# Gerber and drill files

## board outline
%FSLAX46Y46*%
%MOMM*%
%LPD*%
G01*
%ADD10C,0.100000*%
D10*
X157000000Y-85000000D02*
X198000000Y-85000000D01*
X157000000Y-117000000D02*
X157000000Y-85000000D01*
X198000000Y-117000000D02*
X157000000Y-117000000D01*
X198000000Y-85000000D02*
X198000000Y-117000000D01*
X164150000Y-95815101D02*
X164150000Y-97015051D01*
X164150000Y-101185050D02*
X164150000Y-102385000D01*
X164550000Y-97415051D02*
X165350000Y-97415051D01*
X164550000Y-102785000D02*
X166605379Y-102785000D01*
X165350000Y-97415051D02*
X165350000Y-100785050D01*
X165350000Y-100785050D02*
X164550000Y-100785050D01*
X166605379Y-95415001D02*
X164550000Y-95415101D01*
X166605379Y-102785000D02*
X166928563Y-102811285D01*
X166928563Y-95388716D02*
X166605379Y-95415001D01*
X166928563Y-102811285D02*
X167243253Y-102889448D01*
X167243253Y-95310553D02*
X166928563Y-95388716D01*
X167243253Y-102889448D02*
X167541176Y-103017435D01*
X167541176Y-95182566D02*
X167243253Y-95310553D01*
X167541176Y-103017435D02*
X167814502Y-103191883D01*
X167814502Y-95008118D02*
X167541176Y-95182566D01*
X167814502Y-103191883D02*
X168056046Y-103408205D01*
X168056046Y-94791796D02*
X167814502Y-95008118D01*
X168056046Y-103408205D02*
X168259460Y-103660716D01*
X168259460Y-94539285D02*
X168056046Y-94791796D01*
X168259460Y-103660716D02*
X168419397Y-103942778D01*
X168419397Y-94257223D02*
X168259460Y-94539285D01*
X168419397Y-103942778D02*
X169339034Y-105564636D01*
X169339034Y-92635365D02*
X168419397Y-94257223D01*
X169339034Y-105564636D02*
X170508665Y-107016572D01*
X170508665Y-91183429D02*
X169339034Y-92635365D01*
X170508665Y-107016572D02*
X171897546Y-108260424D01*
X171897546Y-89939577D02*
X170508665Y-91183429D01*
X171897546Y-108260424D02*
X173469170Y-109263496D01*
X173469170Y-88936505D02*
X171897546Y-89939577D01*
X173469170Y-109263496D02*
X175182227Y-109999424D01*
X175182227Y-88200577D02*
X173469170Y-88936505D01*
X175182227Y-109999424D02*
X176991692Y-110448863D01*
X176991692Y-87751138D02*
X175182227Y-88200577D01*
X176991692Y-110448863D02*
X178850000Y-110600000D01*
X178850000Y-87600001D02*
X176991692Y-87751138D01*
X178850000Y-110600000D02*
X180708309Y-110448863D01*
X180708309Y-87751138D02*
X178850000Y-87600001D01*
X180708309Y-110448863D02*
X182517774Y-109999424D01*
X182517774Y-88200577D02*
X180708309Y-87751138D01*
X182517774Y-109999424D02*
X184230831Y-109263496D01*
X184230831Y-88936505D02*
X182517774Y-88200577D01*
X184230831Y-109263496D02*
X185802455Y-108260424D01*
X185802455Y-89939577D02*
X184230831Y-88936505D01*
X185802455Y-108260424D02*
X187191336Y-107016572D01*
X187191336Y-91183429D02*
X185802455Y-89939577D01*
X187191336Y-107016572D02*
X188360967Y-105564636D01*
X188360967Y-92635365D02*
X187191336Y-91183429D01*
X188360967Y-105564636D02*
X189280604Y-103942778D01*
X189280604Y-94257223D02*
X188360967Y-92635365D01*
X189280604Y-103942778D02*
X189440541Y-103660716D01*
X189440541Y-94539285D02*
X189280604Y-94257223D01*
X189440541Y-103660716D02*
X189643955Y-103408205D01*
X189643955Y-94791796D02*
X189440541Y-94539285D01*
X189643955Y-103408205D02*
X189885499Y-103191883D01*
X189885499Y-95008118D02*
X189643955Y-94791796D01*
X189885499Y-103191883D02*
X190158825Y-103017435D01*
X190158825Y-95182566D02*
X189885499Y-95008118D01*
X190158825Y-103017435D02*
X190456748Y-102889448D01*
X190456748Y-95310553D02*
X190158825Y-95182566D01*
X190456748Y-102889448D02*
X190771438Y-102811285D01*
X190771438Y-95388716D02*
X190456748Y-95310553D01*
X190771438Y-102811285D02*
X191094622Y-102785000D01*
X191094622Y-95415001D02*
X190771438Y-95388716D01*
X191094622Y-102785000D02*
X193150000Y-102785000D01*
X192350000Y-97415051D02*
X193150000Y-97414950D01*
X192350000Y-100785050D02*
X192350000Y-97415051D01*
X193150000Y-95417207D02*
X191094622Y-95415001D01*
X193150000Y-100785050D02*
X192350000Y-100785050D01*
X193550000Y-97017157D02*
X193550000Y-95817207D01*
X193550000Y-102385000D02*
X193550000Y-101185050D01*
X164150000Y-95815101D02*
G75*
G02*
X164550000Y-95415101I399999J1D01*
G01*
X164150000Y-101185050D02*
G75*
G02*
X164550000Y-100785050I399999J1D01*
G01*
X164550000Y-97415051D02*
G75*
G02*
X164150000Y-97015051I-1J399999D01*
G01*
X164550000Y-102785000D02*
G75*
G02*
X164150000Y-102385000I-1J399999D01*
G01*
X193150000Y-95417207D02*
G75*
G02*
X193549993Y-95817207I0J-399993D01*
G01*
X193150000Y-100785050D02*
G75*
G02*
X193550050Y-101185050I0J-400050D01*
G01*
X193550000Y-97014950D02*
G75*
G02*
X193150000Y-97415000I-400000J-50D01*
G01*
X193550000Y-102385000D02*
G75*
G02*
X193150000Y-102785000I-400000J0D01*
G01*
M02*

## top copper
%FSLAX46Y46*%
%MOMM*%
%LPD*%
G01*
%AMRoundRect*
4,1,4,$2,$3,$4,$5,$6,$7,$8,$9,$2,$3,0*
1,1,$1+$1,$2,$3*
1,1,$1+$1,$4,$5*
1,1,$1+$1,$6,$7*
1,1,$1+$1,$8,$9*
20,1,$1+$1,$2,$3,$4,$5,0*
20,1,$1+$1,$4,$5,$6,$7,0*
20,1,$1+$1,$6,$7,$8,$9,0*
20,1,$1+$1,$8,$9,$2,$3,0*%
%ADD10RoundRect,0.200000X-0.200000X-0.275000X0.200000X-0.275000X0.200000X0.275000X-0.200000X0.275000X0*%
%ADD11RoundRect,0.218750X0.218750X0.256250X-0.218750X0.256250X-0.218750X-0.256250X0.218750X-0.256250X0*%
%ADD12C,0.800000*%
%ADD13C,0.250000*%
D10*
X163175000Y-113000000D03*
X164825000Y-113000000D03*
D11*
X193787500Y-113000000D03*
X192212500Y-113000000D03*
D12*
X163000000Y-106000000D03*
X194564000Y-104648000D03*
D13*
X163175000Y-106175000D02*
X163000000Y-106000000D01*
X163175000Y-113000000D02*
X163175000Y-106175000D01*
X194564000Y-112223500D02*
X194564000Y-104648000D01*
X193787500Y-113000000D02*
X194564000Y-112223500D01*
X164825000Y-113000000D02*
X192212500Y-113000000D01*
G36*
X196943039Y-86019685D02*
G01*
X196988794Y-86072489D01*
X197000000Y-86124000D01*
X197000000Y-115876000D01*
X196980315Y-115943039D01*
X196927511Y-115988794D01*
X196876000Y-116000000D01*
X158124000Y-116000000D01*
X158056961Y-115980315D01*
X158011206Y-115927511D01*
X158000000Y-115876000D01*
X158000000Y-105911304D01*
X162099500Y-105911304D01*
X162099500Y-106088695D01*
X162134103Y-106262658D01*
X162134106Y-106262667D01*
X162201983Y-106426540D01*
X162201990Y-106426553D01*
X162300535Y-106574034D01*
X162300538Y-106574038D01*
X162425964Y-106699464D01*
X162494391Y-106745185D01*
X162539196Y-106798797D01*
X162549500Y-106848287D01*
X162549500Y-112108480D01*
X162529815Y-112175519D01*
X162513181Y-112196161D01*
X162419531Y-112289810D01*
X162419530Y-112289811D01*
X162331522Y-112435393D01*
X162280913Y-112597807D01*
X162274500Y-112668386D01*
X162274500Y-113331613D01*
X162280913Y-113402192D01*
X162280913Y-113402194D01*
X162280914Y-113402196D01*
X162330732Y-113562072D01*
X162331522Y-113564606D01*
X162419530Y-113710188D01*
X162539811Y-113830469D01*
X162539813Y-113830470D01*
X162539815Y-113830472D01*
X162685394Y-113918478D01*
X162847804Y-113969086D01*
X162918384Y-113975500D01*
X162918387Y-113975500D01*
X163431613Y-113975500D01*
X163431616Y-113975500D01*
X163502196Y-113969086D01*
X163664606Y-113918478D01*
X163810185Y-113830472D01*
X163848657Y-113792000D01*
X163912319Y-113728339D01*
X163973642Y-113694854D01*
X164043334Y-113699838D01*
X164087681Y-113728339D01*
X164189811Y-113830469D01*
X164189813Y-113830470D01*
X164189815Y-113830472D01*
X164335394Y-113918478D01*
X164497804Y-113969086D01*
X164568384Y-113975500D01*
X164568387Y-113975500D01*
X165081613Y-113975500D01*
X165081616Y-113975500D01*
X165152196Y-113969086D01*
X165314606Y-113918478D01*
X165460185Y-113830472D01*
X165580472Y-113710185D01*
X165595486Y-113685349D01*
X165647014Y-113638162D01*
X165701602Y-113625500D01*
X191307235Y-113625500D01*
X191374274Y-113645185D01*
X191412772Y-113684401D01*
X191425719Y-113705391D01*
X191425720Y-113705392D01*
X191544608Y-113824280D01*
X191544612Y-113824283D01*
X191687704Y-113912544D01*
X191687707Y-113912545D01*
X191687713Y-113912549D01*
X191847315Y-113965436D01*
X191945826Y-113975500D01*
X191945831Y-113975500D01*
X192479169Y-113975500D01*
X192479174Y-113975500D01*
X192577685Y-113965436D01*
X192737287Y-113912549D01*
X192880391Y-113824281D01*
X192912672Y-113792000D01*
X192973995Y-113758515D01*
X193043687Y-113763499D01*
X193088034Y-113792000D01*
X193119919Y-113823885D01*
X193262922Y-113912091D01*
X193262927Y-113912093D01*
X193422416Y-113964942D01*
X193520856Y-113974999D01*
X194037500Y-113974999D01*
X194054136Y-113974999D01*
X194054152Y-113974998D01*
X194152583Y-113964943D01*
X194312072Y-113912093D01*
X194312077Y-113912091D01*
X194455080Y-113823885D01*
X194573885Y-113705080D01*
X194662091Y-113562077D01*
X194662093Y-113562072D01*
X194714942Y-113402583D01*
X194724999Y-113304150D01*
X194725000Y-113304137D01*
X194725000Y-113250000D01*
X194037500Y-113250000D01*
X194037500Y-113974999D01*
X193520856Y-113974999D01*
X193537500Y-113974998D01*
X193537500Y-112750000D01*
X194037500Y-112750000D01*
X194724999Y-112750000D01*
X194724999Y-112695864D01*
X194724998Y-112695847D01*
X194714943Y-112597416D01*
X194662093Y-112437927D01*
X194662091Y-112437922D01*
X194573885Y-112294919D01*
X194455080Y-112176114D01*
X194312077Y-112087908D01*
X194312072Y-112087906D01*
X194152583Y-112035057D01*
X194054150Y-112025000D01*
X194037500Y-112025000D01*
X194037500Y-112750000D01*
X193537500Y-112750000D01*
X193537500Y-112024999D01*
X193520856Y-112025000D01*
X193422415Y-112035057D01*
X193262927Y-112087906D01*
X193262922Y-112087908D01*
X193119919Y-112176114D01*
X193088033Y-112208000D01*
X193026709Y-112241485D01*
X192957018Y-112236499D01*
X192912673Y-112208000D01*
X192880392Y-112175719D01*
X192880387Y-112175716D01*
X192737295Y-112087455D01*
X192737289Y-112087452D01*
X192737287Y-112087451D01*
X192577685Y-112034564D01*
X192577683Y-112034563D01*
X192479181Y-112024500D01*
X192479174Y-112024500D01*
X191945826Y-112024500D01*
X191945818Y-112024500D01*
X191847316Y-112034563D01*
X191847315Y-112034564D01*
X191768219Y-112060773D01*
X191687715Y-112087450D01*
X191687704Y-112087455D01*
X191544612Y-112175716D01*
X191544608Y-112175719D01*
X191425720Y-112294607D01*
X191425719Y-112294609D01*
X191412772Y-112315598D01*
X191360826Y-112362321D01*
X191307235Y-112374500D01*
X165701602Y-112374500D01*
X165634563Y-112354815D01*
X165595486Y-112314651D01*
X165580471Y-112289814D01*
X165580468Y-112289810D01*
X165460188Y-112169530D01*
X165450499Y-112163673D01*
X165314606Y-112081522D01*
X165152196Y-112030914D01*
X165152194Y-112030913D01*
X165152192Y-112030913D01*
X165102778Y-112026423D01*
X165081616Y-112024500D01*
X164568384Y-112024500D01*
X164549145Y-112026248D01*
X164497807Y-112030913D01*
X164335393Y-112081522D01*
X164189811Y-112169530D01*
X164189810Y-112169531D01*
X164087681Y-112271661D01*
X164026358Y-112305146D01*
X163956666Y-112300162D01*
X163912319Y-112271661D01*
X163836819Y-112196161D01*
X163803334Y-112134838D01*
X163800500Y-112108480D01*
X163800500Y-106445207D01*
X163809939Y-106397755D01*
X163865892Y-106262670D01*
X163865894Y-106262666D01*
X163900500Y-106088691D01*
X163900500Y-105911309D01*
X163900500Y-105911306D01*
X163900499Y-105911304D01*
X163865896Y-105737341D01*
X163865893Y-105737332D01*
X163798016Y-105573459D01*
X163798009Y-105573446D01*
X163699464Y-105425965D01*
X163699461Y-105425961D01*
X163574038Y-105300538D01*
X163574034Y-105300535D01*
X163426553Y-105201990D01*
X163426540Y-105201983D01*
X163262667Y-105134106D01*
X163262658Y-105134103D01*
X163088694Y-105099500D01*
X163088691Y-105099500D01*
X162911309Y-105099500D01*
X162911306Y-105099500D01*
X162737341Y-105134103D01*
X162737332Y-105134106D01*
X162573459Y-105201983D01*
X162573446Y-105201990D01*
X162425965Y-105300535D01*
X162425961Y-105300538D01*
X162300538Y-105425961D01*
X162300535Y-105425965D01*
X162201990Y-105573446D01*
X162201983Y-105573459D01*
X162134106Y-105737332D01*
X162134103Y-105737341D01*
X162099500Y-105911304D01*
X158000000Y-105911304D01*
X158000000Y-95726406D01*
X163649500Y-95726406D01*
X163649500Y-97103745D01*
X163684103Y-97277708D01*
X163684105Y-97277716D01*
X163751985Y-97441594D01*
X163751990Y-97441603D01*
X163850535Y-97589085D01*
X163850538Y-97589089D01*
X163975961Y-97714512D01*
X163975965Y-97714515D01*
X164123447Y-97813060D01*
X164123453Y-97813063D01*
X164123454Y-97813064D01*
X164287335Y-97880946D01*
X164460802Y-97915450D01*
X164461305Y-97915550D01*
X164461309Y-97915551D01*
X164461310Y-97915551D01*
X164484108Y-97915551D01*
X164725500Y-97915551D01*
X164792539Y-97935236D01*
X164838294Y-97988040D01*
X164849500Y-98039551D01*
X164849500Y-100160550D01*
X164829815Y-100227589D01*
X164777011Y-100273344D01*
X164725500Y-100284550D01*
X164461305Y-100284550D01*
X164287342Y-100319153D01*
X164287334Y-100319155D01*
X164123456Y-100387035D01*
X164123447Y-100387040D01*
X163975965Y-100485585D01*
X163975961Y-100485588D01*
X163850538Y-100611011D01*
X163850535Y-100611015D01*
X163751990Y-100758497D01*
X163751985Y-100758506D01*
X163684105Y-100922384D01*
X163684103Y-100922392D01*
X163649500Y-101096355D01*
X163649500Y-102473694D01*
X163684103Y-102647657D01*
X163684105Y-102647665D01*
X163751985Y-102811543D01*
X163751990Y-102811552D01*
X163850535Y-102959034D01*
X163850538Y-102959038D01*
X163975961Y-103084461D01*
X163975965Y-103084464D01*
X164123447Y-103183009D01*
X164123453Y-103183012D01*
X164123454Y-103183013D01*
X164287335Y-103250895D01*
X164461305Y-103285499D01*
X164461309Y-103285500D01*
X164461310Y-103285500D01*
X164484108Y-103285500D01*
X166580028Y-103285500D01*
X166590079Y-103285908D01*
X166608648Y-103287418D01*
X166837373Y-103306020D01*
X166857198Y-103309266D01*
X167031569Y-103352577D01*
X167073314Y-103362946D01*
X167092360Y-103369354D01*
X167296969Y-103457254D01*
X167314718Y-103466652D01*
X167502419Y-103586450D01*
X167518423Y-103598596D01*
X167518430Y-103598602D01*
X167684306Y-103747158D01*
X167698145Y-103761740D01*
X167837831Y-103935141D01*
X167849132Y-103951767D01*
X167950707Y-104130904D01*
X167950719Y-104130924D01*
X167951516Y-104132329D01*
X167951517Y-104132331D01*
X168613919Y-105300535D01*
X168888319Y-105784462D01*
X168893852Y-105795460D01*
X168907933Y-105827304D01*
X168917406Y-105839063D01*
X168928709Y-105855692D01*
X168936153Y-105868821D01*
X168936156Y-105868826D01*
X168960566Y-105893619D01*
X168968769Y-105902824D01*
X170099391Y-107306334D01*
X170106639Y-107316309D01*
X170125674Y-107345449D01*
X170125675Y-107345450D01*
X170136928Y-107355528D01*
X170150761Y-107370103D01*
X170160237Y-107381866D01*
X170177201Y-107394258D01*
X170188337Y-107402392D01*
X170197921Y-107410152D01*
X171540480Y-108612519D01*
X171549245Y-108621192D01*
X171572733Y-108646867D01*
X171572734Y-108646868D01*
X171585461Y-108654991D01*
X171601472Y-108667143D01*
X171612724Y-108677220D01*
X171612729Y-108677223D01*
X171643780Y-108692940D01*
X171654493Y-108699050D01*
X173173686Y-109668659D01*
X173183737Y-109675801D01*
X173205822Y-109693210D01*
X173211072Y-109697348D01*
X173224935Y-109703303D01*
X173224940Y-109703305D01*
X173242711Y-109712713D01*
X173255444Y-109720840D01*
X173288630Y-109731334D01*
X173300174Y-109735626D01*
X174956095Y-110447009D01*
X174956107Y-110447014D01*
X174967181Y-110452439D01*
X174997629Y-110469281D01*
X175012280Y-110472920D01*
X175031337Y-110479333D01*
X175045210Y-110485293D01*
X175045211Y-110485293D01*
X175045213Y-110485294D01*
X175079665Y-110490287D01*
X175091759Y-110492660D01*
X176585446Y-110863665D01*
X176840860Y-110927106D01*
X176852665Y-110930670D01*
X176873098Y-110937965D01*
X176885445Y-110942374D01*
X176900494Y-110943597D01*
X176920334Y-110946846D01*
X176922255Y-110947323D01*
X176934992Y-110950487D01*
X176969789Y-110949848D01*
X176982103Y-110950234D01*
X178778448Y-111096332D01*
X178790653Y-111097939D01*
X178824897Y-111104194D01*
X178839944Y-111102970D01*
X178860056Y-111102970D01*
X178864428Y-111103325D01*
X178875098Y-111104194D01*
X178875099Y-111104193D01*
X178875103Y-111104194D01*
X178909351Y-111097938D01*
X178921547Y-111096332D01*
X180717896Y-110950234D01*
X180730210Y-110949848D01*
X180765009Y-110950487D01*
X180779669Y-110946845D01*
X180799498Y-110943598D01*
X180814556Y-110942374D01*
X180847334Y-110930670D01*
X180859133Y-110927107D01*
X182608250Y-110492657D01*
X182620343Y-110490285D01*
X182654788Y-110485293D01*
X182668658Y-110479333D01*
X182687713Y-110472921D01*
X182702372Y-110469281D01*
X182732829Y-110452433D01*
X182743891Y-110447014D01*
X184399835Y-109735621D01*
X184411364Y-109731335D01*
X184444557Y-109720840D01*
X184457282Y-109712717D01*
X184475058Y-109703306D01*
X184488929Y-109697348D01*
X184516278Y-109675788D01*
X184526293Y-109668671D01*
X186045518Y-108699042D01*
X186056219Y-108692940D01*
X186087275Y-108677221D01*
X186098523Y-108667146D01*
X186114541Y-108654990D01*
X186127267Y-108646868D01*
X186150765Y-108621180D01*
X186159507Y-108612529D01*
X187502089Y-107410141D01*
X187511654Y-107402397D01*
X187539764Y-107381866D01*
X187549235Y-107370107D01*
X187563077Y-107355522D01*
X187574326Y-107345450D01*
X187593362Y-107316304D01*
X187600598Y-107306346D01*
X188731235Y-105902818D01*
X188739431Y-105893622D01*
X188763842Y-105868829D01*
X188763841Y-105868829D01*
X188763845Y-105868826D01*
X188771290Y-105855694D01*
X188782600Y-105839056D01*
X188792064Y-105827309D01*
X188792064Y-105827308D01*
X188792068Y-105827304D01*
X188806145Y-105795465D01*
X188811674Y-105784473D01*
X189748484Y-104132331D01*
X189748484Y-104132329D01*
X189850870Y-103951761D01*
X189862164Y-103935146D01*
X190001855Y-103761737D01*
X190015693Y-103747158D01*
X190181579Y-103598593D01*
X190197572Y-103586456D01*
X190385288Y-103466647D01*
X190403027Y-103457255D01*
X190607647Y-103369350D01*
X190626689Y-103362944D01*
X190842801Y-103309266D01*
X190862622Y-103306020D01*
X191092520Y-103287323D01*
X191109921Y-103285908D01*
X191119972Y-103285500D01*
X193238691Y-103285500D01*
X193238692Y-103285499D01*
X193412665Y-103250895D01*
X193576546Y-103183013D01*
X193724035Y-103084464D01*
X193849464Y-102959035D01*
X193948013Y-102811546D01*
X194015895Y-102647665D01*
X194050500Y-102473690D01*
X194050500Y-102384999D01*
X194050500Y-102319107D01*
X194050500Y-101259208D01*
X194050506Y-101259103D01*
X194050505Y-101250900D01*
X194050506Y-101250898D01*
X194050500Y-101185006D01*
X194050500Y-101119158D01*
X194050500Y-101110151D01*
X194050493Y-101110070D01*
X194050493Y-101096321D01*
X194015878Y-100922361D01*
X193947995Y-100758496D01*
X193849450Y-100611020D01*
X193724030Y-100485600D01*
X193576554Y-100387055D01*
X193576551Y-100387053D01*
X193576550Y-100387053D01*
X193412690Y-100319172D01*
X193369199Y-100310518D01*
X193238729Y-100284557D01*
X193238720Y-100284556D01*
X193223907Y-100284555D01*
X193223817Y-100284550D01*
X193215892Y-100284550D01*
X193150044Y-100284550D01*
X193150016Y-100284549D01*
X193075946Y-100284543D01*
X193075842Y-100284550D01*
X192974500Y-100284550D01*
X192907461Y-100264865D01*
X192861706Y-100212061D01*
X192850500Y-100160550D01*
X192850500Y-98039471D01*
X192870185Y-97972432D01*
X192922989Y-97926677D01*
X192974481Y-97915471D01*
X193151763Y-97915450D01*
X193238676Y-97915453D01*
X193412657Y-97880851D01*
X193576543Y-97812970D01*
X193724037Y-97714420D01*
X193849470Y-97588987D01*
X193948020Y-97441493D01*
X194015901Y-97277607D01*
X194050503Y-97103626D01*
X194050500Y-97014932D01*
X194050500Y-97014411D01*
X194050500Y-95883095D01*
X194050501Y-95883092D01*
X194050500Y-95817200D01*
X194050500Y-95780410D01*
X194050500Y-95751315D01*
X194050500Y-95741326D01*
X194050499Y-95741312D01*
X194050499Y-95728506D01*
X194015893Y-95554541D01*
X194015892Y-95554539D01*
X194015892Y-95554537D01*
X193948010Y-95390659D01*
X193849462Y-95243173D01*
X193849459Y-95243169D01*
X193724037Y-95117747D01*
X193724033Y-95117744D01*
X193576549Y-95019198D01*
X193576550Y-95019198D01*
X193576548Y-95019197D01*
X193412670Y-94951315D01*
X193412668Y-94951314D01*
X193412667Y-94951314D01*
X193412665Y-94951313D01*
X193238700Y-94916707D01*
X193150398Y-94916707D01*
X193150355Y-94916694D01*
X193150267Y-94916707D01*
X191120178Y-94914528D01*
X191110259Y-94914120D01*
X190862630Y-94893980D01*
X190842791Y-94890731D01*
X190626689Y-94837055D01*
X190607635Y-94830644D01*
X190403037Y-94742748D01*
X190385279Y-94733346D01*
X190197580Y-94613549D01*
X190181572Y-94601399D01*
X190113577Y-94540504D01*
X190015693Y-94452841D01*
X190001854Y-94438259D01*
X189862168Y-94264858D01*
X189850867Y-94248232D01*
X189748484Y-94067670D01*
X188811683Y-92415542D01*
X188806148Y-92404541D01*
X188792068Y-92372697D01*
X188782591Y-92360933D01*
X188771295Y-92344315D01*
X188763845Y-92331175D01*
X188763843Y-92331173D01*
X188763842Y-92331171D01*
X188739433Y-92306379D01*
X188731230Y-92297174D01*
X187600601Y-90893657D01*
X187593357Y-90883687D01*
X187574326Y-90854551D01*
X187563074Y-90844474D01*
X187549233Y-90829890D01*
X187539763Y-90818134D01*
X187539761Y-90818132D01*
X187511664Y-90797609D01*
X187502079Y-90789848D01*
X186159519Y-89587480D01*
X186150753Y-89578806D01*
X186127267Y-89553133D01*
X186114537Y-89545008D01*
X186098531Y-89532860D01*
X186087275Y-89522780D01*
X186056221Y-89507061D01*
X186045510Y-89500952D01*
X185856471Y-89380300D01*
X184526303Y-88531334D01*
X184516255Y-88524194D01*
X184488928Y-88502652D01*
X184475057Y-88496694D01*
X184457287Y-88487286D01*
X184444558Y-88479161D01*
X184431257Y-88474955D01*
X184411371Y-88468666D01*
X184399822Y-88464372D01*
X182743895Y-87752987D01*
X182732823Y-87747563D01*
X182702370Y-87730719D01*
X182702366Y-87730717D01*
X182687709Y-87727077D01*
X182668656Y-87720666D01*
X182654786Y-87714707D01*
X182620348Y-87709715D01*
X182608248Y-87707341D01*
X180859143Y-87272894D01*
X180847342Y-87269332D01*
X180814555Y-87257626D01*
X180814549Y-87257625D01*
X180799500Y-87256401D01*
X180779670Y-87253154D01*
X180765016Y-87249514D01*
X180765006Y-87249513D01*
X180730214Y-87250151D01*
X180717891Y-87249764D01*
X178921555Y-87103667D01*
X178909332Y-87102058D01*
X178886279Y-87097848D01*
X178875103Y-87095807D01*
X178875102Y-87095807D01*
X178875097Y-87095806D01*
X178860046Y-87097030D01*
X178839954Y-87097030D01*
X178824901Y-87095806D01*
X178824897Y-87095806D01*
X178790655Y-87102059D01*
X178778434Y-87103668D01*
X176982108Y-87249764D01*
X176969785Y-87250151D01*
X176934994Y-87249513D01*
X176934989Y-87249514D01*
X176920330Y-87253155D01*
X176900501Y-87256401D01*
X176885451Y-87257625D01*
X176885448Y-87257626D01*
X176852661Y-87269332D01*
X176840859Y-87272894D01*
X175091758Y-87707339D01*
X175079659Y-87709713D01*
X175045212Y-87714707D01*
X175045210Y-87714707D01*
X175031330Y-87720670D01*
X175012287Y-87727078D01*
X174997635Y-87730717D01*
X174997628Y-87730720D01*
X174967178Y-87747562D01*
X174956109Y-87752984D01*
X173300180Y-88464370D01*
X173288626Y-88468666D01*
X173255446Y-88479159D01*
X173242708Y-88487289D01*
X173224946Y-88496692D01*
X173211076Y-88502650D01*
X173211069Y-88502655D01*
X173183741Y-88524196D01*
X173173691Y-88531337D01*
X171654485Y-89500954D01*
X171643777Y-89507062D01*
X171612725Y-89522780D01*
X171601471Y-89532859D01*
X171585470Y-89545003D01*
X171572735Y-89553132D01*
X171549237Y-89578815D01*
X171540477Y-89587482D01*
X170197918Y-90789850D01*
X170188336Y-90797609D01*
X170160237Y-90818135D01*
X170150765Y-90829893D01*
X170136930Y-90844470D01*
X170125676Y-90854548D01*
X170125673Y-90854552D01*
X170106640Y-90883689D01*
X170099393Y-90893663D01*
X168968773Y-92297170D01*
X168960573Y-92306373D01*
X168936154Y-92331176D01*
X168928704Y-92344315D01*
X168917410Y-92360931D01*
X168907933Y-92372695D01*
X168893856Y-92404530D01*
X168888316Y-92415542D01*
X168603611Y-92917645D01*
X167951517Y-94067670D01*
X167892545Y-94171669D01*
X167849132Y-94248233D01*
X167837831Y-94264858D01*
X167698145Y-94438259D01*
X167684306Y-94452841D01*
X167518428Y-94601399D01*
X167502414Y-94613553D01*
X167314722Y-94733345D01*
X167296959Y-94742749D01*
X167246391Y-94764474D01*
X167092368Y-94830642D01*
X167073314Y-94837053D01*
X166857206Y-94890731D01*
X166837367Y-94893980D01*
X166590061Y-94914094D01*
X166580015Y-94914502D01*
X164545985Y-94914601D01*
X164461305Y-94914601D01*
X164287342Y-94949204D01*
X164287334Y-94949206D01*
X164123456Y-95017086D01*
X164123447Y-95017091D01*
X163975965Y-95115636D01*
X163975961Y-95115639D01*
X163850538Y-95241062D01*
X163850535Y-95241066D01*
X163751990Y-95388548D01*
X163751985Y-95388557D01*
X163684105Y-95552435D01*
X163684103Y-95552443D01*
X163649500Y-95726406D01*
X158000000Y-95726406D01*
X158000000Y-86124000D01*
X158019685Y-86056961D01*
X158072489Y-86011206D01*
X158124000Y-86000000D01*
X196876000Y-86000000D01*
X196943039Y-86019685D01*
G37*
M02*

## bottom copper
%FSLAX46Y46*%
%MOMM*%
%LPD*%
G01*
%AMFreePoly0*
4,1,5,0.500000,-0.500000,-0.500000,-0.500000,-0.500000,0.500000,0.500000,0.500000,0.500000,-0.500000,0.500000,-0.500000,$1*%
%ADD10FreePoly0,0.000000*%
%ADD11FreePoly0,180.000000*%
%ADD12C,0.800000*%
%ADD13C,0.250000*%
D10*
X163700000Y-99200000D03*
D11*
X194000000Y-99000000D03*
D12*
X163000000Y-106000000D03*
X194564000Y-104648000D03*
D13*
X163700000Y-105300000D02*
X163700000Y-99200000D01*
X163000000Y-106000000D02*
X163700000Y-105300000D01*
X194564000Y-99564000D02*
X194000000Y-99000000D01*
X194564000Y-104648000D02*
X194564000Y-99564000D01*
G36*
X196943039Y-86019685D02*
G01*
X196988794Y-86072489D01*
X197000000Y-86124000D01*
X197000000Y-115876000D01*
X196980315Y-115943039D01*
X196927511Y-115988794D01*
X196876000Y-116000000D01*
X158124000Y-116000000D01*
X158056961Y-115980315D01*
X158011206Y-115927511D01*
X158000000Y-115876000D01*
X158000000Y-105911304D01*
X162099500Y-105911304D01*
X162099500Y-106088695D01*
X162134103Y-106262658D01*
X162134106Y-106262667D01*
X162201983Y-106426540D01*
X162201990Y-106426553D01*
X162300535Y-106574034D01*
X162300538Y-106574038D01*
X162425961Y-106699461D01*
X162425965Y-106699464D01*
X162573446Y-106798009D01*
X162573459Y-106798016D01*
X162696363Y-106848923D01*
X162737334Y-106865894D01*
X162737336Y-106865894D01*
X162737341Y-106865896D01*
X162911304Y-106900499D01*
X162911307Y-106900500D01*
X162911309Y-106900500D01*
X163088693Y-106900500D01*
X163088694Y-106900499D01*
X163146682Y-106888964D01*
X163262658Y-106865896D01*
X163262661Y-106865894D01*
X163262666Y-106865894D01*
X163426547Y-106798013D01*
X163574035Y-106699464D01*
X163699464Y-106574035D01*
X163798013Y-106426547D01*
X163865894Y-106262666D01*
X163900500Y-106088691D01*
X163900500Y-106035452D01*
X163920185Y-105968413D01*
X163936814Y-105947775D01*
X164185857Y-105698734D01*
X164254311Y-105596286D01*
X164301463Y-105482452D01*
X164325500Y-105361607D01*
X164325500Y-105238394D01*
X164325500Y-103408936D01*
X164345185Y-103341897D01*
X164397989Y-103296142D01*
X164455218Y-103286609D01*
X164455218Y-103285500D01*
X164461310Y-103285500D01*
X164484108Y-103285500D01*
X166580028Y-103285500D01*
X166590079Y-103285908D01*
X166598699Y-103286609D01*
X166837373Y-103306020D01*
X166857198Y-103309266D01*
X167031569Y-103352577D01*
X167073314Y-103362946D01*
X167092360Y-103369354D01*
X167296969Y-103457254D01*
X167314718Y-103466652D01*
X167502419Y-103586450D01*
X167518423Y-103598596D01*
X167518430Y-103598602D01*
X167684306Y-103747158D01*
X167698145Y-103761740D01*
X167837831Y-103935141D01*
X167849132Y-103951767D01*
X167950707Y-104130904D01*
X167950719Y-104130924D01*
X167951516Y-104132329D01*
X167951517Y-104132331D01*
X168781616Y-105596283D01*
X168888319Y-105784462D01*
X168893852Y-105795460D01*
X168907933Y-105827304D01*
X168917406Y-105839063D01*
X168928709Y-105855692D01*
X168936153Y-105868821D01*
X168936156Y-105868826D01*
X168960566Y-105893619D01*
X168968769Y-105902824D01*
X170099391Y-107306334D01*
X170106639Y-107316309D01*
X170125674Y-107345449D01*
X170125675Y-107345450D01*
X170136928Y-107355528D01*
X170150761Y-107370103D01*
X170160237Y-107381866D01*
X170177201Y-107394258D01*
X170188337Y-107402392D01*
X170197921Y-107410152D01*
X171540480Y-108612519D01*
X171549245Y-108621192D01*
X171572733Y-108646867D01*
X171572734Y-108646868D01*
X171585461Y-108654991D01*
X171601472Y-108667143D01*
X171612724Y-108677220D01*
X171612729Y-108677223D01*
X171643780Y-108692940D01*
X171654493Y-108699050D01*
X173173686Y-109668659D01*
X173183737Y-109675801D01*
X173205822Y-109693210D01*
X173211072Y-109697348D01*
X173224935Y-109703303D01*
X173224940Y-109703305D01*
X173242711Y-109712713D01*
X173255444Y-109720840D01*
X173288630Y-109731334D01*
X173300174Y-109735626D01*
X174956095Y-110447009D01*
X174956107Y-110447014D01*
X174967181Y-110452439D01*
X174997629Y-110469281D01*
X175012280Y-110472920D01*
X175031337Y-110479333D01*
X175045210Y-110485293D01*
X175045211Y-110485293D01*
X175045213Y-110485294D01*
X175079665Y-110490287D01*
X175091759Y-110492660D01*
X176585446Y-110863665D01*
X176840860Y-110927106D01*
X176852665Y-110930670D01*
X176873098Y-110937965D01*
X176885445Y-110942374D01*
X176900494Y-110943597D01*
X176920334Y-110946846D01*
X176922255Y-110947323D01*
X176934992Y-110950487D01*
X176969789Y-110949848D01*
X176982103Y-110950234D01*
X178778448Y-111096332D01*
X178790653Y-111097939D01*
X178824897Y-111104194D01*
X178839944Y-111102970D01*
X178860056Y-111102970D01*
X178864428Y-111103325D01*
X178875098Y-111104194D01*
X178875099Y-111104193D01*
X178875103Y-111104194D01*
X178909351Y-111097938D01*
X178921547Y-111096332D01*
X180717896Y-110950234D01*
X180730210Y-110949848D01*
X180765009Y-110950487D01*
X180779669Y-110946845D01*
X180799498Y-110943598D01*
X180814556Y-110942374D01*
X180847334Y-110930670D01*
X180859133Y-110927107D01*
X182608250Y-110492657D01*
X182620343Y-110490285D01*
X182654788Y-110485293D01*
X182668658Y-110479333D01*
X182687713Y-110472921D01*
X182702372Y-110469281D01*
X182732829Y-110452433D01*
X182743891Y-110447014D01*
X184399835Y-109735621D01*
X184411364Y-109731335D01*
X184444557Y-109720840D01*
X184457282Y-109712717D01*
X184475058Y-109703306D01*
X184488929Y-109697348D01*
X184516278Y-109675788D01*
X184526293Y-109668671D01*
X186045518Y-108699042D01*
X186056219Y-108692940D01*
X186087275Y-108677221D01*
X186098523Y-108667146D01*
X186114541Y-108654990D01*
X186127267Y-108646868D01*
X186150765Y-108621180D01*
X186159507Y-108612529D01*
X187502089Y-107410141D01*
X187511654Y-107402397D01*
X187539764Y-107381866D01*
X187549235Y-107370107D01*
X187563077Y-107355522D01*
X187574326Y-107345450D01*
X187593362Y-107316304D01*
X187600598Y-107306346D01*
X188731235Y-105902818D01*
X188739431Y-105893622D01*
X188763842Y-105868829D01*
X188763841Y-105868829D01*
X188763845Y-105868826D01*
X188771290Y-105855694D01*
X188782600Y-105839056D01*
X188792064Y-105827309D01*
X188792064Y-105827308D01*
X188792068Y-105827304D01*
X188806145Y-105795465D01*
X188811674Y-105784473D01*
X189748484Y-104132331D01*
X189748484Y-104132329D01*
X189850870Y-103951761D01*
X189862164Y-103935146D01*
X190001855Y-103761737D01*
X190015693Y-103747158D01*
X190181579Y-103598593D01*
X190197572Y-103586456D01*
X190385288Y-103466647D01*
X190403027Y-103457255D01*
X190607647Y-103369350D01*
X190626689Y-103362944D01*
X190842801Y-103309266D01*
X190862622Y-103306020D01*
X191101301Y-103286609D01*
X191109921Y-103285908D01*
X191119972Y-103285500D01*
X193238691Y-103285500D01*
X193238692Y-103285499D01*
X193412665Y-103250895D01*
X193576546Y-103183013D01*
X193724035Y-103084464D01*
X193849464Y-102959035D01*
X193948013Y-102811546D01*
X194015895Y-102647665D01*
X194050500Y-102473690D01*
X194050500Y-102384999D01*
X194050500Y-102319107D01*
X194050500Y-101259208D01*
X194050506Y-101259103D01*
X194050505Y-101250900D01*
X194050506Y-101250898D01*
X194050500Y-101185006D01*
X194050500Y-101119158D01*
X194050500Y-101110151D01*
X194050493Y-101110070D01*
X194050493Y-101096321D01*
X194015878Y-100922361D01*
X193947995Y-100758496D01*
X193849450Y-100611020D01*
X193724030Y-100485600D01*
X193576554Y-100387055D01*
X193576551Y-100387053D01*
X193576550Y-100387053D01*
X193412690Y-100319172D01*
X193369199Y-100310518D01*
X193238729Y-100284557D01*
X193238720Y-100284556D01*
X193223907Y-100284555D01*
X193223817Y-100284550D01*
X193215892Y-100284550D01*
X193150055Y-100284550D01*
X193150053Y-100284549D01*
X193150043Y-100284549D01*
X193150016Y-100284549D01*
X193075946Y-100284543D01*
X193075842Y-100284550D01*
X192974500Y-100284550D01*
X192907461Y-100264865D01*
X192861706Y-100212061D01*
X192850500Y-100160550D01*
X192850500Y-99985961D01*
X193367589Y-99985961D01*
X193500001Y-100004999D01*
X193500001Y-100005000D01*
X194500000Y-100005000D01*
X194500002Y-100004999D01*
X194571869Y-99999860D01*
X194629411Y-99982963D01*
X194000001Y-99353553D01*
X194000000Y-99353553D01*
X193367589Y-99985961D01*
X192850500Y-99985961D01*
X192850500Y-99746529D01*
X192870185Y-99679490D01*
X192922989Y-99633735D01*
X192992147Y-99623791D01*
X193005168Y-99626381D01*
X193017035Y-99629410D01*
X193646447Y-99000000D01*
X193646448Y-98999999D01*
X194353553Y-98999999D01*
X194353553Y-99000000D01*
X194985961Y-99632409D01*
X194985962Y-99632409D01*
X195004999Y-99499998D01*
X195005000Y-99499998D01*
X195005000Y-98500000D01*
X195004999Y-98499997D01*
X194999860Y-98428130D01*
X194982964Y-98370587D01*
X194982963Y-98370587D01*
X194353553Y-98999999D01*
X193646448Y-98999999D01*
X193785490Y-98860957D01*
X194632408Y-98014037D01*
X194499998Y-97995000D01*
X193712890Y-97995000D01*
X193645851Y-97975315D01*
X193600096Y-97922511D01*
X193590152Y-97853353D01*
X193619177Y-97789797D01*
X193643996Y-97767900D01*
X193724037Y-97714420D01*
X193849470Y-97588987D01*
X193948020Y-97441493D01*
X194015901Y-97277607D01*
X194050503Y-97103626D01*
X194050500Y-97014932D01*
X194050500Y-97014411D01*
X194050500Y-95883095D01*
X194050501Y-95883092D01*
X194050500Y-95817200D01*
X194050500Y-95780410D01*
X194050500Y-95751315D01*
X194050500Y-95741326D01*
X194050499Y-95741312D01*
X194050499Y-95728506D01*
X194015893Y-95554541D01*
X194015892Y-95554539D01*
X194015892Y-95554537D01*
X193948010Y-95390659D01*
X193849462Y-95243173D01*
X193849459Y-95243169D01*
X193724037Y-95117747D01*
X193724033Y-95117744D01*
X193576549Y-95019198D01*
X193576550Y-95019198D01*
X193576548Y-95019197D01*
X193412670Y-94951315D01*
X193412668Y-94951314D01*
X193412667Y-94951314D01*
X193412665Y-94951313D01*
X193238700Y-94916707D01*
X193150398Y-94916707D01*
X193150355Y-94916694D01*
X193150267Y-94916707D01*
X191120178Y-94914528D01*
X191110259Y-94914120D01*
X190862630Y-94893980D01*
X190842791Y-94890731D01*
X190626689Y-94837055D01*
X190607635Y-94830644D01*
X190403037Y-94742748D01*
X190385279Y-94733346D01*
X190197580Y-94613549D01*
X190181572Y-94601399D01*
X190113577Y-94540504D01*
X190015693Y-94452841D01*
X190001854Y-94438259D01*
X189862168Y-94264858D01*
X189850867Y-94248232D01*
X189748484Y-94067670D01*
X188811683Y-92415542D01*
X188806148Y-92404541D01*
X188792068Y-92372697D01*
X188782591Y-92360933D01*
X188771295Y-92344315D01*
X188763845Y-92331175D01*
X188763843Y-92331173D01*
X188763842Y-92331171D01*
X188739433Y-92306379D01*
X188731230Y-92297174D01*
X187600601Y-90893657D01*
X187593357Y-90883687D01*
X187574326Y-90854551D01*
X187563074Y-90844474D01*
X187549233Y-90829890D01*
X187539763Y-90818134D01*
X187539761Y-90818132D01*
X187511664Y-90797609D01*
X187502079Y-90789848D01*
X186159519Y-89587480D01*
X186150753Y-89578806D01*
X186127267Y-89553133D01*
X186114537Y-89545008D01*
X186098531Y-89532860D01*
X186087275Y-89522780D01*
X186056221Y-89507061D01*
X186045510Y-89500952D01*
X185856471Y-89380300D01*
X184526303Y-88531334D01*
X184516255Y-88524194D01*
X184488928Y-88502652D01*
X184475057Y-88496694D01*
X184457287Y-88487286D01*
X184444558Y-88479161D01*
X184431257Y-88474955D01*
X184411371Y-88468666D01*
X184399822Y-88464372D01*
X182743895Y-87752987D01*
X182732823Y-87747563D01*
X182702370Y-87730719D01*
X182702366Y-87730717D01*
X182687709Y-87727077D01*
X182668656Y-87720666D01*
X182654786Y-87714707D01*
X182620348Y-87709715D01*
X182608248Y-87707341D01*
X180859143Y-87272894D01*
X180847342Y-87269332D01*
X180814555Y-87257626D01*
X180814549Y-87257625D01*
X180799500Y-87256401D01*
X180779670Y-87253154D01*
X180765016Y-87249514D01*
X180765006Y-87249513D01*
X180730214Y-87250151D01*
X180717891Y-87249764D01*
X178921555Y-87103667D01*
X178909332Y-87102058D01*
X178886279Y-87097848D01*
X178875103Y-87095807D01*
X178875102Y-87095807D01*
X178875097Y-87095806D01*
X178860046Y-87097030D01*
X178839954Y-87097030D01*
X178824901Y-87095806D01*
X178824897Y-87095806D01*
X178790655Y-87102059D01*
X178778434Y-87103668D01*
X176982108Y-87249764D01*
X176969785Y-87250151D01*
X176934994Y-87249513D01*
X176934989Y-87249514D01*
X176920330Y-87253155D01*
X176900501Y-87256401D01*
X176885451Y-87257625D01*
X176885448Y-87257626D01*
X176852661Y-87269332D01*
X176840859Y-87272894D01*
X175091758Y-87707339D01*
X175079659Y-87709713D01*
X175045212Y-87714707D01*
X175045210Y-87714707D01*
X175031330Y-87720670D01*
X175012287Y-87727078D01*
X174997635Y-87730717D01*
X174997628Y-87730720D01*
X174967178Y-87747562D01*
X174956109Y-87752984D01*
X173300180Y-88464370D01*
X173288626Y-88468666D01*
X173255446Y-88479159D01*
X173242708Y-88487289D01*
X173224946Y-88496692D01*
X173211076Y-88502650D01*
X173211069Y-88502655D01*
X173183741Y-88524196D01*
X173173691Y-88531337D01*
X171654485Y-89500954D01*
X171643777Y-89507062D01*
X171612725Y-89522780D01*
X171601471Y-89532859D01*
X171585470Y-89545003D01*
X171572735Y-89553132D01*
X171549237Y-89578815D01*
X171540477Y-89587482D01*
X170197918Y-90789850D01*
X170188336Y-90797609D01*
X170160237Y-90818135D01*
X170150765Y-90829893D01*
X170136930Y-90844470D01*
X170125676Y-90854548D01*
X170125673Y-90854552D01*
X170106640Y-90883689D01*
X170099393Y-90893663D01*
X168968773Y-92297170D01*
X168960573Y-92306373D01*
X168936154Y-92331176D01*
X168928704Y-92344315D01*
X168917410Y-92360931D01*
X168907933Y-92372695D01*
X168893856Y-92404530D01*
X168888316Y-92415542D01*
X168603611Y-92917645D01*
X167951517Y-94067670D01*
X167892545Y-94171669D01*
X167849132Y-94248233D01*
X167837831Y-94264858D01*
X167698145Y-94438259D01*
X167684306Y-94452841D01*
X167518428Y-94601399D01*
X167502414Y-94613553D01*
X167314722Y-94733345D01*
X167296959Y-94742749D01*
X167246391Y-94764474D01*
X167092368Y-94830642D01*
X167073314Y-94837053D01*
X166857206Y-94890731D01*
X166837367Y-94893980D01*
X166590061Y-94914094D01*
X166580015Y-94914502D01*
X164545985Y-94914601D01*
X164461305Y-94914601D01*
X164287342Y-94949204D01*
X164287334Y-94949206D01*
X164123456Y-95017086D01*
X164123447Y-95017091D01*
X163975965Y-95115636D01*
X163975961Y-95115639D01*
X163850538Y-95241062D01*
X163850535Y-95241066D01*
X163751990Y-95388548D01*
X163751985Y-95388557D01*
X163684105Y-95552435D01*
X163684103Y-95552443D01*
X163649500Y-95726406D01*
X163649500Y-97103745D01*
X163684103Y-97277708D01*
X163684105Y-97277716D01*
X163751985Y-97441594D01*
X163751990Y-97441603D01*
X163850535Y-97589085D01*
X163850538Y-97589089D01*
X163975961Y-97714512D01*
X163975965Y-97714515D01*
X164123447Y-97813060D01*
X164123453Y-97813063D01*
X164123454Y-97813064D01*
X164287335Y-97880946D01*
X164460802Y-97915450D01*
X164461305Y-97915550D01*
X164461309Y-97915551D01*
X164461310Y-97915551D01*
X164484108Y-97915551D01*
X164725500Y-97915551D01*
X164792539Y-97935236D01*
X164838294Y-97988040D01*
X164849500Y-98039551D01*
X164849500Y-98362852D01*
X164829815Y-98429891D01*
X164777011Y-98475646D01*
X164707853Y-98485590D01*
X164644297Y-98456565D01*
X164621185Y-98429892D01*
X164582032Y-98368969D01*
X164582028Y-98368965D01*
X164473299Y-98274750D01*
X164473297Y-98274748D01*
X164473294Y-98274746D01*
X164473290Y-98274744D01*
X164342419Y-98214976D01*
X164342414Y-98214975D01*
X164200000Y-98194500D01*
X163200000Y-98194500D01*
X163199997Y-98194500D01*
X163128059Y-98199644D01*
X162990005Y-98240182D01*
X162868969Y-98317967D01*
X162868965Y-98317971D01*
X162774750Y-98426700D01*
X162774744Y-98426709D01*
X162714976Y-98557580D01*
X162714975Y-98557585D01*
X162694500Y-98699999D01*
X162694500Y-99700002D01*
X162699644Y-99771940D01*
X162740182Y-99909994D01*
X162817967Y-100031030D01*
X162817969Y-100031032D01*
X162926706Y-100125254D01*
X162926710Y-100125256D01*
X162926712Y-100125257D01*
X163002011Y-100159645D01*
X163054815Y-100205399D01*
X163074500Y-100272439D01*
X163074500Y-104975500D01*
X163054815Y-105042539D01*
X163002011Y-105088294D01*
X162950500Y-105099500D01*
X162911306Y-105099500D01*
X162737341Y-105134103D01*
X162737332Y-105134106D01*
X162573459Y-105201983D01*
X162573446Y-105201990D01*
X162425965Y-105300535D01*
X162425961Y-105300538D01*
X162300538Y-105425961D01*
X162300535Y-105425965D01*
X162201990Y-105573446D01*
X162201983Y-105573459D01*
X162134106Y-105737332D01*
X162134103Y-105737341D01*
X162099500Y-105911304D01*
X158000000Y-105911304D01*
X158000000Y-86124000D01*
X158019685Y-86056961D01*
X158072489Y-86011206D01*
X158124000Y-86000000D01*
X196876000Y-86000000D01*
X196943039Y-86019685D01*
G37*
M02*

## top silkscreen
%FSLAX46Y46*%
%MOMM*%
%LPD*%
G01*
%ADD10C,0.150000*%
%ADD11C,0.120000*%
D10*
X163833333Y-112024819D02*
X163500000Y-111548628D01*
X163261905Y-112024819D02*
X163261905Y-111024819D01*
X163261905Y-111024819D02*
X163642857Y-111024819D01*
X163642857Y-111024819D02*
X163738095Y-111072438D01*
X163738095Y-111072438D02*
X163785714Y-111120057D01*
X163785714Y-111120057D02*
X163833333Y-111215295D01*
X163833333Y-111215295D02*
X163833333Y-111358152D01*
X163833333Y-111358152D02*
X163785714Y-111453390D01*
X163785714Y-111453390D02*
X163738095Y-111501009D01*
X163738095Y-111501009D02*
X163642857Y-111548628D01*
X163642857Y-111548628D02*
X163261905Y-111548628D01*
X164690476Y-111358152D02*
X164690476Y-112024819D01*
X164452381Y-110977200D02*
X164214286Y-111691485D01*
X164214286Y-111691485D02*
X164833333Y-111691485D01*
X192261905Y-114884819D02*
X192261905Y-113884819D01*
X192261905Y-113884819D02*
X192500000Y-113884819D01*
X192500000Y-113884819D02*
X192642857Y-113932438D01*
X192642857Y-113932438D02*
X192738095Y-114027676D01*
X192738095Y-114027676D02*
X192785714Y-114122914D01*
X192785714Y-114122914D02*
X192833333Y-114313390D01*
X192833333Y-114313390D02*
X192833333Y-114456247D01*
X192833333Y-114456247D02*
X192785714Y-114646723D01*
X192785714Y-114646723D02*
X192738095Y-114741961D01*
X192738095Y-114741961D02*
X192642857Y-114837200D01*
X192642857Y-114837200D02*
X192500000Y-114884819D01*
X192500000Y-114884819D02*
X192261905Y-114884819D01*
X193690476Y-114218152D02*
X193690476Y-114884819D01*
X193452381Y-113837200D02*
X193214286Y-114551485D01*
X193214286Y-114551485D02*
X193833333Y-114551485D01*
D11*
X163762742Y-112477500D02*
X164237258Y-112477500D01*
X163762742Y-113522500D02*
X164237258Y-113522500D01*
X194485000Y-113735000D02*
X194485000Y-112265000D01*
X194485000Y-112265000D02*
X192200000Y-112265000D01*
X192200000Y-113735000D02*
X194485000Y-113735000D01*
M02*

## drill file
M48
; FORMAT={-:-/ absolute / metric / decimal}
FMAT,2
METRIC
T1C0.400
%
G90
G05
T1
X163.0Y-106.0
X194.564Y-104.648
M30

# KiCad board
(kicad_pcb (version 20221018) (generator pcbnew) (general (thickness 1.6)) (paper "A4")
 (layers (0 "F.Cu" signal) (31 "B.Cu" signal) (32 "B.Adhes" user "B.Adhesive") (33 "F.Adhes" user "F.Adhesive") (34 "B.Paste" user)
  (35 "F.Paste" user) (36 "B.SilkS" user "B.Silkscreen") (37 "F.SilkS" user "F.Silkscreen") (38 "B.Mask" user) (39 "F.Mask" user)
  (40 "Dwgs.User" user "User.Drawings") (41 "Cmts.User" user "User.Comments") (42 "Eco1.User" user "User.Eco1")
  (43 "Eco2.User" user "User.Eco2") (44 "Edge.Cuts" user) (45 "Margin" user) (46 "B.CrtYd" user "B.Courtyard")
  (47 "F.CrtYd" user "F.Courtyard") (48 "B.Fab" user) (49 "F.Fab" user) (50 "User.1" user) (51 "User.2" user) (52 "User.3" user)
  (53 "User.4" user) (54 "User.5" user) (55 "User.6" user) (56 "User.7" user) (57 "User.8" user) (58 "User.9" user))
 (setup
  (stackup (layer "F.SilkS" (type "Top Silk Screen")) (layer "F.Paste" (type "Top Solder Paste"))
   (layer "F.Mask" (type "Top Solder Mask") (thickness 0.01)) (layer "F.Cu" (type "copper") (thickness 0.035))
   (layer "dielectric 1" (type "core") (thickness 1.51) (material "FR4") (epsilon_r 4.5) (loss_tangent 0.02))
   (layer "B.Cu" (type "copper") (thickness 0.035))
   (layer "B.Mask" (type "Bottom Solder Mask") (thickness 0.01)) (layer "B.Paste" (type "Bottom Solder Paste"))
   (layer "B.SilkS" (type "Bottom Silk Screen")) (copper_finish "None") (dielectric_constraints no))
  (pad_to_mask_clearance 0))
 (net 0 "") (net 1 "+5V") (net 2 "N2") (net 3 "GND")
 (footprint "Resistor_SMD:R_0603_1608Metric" (layer "F.Cu") (at 164 113)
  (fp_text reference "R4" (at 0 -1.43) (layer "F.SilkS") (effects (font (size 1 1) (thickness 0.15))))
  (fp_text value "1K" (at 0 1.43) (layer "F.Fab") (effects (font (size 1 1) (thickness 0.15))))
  (fp_line (start -0.237258 -0.5225) (end 0.237258 -0.5225) (stroke (width 0.12) (type solid)) (layer "F.SilkS"))
  (fp_line (start -0.237258 0.5225) (end 0.237258 0.5225) (stroke (width 0.12) (type solid)) (layer "F.SilkS"))
  (pad "1" smd roundrect (at -0.825 0) (size 0.8 0.95) (layers "F.Cu" "F.Paste" "F.Mask") (roundrect_rratio 0.25) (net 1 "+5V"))
  (pad "2" smd roundrect (at 0.825 0) (size 0.8 0.95) (layers "F.Cu" "F.Paste" "F.Mask") (roundrect_rratio 0.25) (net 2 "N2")))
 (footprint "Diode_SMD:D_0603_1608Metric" (layer "F.Cu") (at 193 113 180)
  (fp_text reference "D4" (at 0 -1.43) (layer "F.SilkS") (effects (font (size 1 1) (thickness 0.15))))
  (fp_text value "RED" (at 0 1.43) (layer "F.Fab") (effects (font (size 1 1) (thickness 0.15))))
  (fp_line (start -1.485 -0.735) (end -1.485 0.735) (stroke (width 0.12) (type solid)) (layer "F.SilkS"))
  (fp_line (start -1.485 0.735) (end 0.8 0.735) (stroke (width 0.12) (type solid)) (layer "F.SilkS"))
  (fp_line (start 0.8 -0.735) (end -1.485 -0.735) (stroke (width 0.12) (type solid)) (layer "F.SilkS"))
  (pad "1" smd roundrect (at -0.7875 0 180) (size 0.875 0.95) (layers "F.Cu" "F.Paste" "F.Mask") (roundrect_rratio 0.25) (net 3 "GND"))
  (pad "2" smd roundrect (at 0.7875 0 180) (size 0.875 0.95) (layers "F.Cu" "F.Paste" "F.Mask") (roundrect_rratio 0.25) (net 2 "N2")))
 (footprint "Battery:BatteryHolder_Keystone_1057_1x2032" (layer "B.Cu") (at 178.85 99.1)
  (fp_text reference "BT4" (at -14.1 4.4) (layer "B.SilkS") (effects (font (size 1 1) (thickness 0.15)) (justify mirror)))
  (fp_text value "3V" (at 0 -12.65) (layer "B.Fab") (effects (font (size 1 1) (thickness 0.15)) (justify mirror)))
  (fp_line (start -14.7 -3.284899) (end -14.7 -2.084949) (stroke (width 0.1) (type solid)) (layer "Edge.Cuts"))
  (fp_line (start -14.7 2.08505) (end -14.7 3.285) (stroke (width 0.1) (type solid)) (layer "Edge.Cuts"))
  (fp_line (start -14.3 -1.684949) (end -13.5 -1.684949) (stroke (width 0.1) (type solid)) (layer "Edge.Cuts"))
  (fp_line (start -14.3 3.685) (end -12.244621 3.685) (stroke (width 0.1) (type solid)) (layer "Edge.Cuts"))
  (fp_line (start -13.5 -1.684949) (end -13.5 1.68505) (stroke (width 0.1) (type solid)) (layer "Edge.Cuts"))
  (fp_line (start -13.5 1.68505) (end -14.3 1.68505) (stroke (width 0.1) (type solid)) (layer "Edge.Cuts"))
  (fp_line (start -12.244621 -3.684999) (end -14.3 -3.684899) (stroke (width 0.1) (type solid)) (layer "Edge.Cuts"))
  (fp_line (start -12.244621 3.685) (end -11.921437 3.711285) (stroke (width 0.1) (type solid)) (layer "Edge.Cuts"))
  (fp_line (start -11.921437 -3.711284) (end -12.244621 -3.684999) (stroke (width 0.1) (type solid)) (layer "Edge.Cuts"))
  (fp_line (start -11.921437 3.711285) (end -11.606747 3.789448) (stroke (width 0.1) (type solid)) (layer "Edge.Cuts"))
  (fp_line (start -11.606747 -3.789447) (end -11.921437 -3.711284) (stroke (width 0.1) (type solid)) (layer "Edge.Cuts"))
  (fp_line (start -11.606747 3.789448) (end -11.308824 3.917435) (stroke (width 0.1) (type solid)) (layer "Edge.Cuts"))
  (fp_line (start -11.308824 -3.917434) (end -11.606747 -3.789447) (stroke (width 0.1) (type solid)) (layer "Edge.Cuts"))
  (fp_line (start -11.308824 3.917435) (end -11.035498 4.091883) (stroke (width 0.1) (type solid)) (layer "Edge.Cuts"))
  (fp_line (start -11.035498 -4.091882) (end -11.308824 -3.917434) (stroke (width 0.1) (type solid)) (layer "Edge.Cuts"))
  (fp_line (start -11.035498 4.091883) (end -10.793954 4.308205) (stroke (width 0.1) (type solid)) (layer "Edge.Cuts"))
  (fp_line (start -10.793954 -4.308204) (end -11.035498 -4.091882) (stroke (width 0.1) (type solid)) (layer "Edge.Cuts"))
  (fp_line (start -10.793954 4.308205) (end -10.59054 4.560716) (stroke (width 0.1) (type solid)) (layer "Edge.Cuts"))
  (fp_line (start -10.59054 -4.560715) (end -10.793954 -4.308204) (stroke (width 0.1) (type solid)) (layer "Edge.Cuts"))
  (fp_line (start -10.59054 4.560716) (end -10.430603 4.842778) (stroke (width 0.1) (type solid)) (layer "Edge.Cuts"))
  (fp_line (start -10.430603 -4.842777) (end -10.59054 -4.560715) (stroke (width 0.1) (type solid)) (layer "Edge.Cuts"))
  (fp_line (start -10.430603 4.842778) (end -9.510966 6.464636) (stroke (width 0.1) (type solid)) (layer "Edge.Cuts"))
  (fp_line (start -9.510966 -6.464635) (end -10.430603 -4.842777) (stroke (width 0.1) (type solid)) (layer "Edge.Cuts"))
  (fp_line (start -9.510966 6.464636) (end -8.341335 7.916572) (stroke (width 0.1) (type solid)) (layer "Edge.Cuts"))
  (fp_line (start -8.341335 -7.916571) (end -9.510966 -6.464635) (stroke (width 0.1) (type solid)) (layer "Edge.Cuts"))
  (fp_line (start -8.341335 7.916572) (end -6.952454 9.160424) (stroke (width 0.1) (type solid)) (layer "Edge.Cuts"))
  (fp_line (start -6.952454 -9.160423) (end -8.341335 -7.916571) (stroke (width 0.1) (type solid)) (layer "Edge.Cuts"))
  (fp_line (start -6.952454 9.160424) (end -5.38083 10.163496) (stroke (width 0.1) (type solid)) (layer "Edge.Cuts"))
  (fp_line (start -5.38083 -10.163495) (end -6.952454 -9.160423) (stroke (width 0.1) (type solid)) (layer "Edge.Cuts"))
  (fp_line (start -5.38083 10.163496) (end -3.667773 10.899424) (stroke (width 0.1) (type solid)) (layer "Edge.Cuts"))
  (fp_line (start -3.667773 -10.899423) (end -5.38083 -10.163495) (stroke (width 0.1) (type solid)) (layer "Edge.Cuts"))
  (fp_line (start -3.667773 10.899424) (end -1.858308 11.348863) (stroke (width 0.1) (type solid)) (layer "Edge.Cuts"))
  (fp_line (start -1.858308 -11.348862) (end -3.667773 -10.899423) (stroke (width 0.1) (type solid)) (layer "Edge.Cuts"))
  (fp_line (start -1.858308 11.348863) (end 0 11.5) (stroke (width 0.1) (type solid)) (layer "Edge.Cuts"))
  (fp_line (start 0 -11.499999) (end -1.858308 -11.348862) (stroke (width 0.1) (type solid)) (layer "Edge.Cuts"))
  (fp_line (start 0 11.5) (end 1.858309 11.348863) (stroke (width 0.1) (type solid)) (layer "Edge.Cuts"))
  (fp_line (start 1.858309 -11.348862) (end 0 -11.499999) (stroke (width 0.1) (type solid)) (layer "Edge.Cuts"))
  (fp_line (start 1.858309 11.348863) (end 3.667774 10.899424) (stroke (width 0.1) (type solid)) (layer "Edge.Cuts"))
  (fp_line (start 3.667774 -10.899423) (end 1.858309 -11.348862) (stroke (width 0.1) (type solid)) (layer "Edge.Cuts"))
  (fp_line (start 3.667774 10.899424) (end 5.380831 10.163496) (stroke (width 0.1) (type solid)) (layer "Edge.Cuts"))
  (fp_line (start 5.380831 -10.163495) (end 3.667774 -10.899423) (stroke (width 0.1) (type solid)) (layer "Edge.Cuts"))
  (fp_line (start 5.380831 10.163496) (end 6.952455 9.160424) (stroke (width 0.1) (type solid)) (layer "Edge.Cuts"))
  (fp_line (start 6.952455 -9.160423) (end 5.380831 -10.163495) (stroke (width 0.1) (type solid)) (layer "Edge.Cuts"))
  (fp_line (start 6.952455 9.160424) (end 8.341336 7.916572) (stroke (width 0.1) (type solid)) (layer "Edge.Cuts"))
  (fp_line (start 8.341336 -7.916571) (end 6.952455 -9.160423) (stroke (width 0.1) (type solid)) (layer "Edge.Cuts"))
  (fp_line (start 8.341336 7.916572) (end 9.510967 6.464636) (stroke (width 0.1) (type solid)) (layer "Edge.Cuts"))
  (fp_line (start 9.510967 -6.464635) (end 8.341336 -7.916571) (stroke (width 0.1) (type solid)) (layer "Edge.Cuts"))
  (fp_line (start 9.510967 6.464636) (end 10.430604 4.842778) (stroke (width 0.1) (type solid)) (layer "Edge.Cuts"))
  (fp_line (start 10.430604 -4.842777) (end 9.510967 -6.464635) (stroke (width 0.1) (type solid)) (layer "Edge.Cuts"))
  (fp_line (start 10.430604 4.842778) (end 10.590541 4.560716) (stroke (width 0.1) (type solid)) (layer "Edge.Cuts"))
  (fp_line (start 10.590541 -4.560715) (end 10.430604 -4.842777) (stroke (width 0.1) (type solid)) (layer "Edge.Cuts"))
  (fp_line (start 10.590541 4.560716) (end 10.793955 4.308205) (stroke (width 0.1) (type solid)) (layer "Edge.Cuts"))
  (fp_line (start 10.793955 -4.308204) (end 10.590541 -4.560715) (stroke (width 0.1) (type solid)) (layer "Edge.Cuts"))
  (fp_line (start 10.793955 4.308205) (end 11.035499 4.091883) (stroke (width 0.1) (type solid)) (layer "Edge.Cuts"))
  (fp_line (start 11.035499 -4.091882) (end 10.793955 -4.308204) (stroke (width 0.1) (type solid)) (layer "Edge.Cuts"))
  (fp_line (start 11.035499 4.091883) (end 11.308825 3.917435) (stroke (width 0.1) (type solid)) (layer "Edge.Cuts"))
  (fp_line (start 11.308825 -3.917434) (end 11.035499 -4.091882) (stroke (width 0.1) (type solid)) (layer "Edge.Cuts"))
  (fp_line (start 11.308825 3.917435) (end 11.606748 3.789448) (stroke (width 0.1) (type solid)) (layer "Edge.Cuts"))
  (fp_line (start 11.606748 -3.789447) (end 11.308825 -3.917434) (stroke (width 0.1) (type solid)) (layer "Edge.Cuts"))
  (fp_line (start 11.606748 3.789448) (end 11.921438 3.711285) (stroke (width 0.1) (type solid)) (layer "Edge.Cuts"))
  (fp_line (start 11.921438 -3.711284) (end 11.606748 -3.789447) (stroke (width 0.1) (type solid)) (layer "Edge.Cuts"))
  (fp_line (start 11.921438 3.711285) (end 12.244622 3.685) (stroke (width 0.1) (type solid)) (layer "Edge.Cuts"))
  (fp_line (start 12.244622 -3.684999) (end 11.921438 -3.711284) (stroke (width 0.1) (type solid)) (layer "Edge.Cuts"))
  (fp_line (start 12.244622 3.685) (end 14.3 3.685) (stroke (width 0.1) (type solid)) (layer "Edge.Cuts"))
  (fp_line (start 13.5 -1.684949) (end 14.3 -1.68505) (stroke (width 0.1) (type solid)) (layer "Edge.Cuts"))
  (fp_line (start 13.5 1.68505) (end 13.5 -1.684949) (stroke (width 0.1) (type solid)) (layer "Edge.Cuts"))
  (fp_line (start 14.3 -3.682793) (end 12.244622 -3.684999) (stroke (width 0.1) (type solid)) (layer "Edge.Cuts"))
  (fp_line (start 14.3 1.68505) (end 13.5 1.68505) (stroke (width 0.1) (type solid)) (layer "Edge.Cuts"))
  (fp_line (start 14.7 -2.082843) (end 14.7 -3.282793) (stroke (width 0.1) (type solid)) (layer "Edge.Cuts"))
  (fp_line (start 14.7 3.285) (end 14.7 2.08505) (stroke (width 0.1) (type solid)) (layer "Edge.Cuts"))
  (fp_arc (start -14.7 -3.284899) (mid -14.582843 -3.567742) (end -14.3 -3.684899) (stroke (width 0.1) (type solid)) (layer "Edge.Cuts"))
  (fp_arc (start -14.7 2.08505) (mid -14.582843 1.802207) (end -14.3 1.68505) (stroke (width 0.1) (type solid)) (layer "Edge.Cuts"))
  (fp_arc (start -14.3 -1.684949) (mid -14.582843 -1.802106) (end -14.7 -2.084949) (stroke (width 0.1) (type solid)) (layer "Edge.Cuts"))
  (fp_arc (start -14.3 3.685) (mid -14.582843 3.567843) (end -14.7 3.285) (stroke (width 0.1) (type solid)) (layer "Edge.Cuts"))
  (fp_arc (start 14.3 -3.682793) (mid 14.58284 -3.565635) (end 14.7 -3.282793) (stroke (width 0.1) (type solid)) (layer "Edge.Cuts"))
  (fp_arc (start 14.3 1.68505) (mid 14.582825 1.80221) (end 14.7 2.08505) (stroke (width 0.1) (type solid)) (layer "Edge.Cuts"))
  (fp_arc (start 14.7 -2.08505) (mid 14.582854 -1.80221) (end 14.3 -1.68505) (stroke (width 0.1) (type solid)) (layer "Edge.Cuts"))
  (fp_arc (start 14.7 3.285) (mid 14.582843 3.567843) (end 14.3 3.685) (stroke (width 0.1) (type solid)) (layer "Edge.Cuts"))
  (pad "1" smd custom (at -15.15 0.1) (size 1 1) (layers "B.Cu" "B.Paste" "B.Mask") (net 1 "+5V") (thermal_bridge_angle 45)
   (options (clearance outline) (anchor rect)) (primitives))
  (pad "2" smd custom (at 15.15 -0.1 180) (size 1 1) (layers "B.Cu" "B.Paste" "B.Mask") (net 3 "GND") (thermal_bridge_angle 45)
   (options (clearance outline) (anchor rect)) (primitives)))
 (gr_line (start 157 85) (end 198 85) (stroke (width 0.1) (type default)) (layer "Edge.Cuts"))
 (gr_line (start 157 117) (end 157 85) (stroke (width 0.1) (type default)) (layer "Edge.Cuts"))
 (gr_line (start 198 117) (end 157 117) (stroke (width 0.1) (type default)) (layer "Edge.Cuts"))
 (gr_line (start 198 85) (end 198 117) (stroke (width 0.1) (type default)) (layer "Edge.Cuts"))
 (segment (start 163.175 106.175) (end 163 106) (width 0.25) (layer "F.Cu") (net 1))
 (segment (start 163.175 113) (end 163.175 106.175) (width 0.25) (layer "F.Cu") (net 1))
 (via (at 163 106) (size 0.8) (drill 0.4) (layers "F.Cu" "B.Cu") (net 1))
 (segment (start 163.7 105.3) (end 163.7 99.2) (width 0.25) (layer "B.Cu") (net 1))
 (segment (start 163 106) (end 163.7 105.3) (width 0.25) (layer "B.Cu") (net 1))
 (segment (start 194.564 112.2235) (end 194.564 104.648) (width 0.25) (layer "F.Cu") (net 3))
 (segment (start 193.7875 113) (end 194.564 112.2235) (width 0.25) (layer "F.Cu") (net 3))
 (via (at 194.564 104.648) (size 0.8) (drill 0.4) (layers "F.Cu" "B.Cu") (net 3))
 (segment (start 194.564 99.564) (end 194 99) (width 0.25) (layer "B.Cu") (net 3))
 (segment (start 194.564 104.648) (end 194.564 99.564) (width 0.25) (layer "B.Cu") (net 3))
 (segment (start 164.825 113) (end 192.2125 113) (width 0.25) (layer "F.Cu") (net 2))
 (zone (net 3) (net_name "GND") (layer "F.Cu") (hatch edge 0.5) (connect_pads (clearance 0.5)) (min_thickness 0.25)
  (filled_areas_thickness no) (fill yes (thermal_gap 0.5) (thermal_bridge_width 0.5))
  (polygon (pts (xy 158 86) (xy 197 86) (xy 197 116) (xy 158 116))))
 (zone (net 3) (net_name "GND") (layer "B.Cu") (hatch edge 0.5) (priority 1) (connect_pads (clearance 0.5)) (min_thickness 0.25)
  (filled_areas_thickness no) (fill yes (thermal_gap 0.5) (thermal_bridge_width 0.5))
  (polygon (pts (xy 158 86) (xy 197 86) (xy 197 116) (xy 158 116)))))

